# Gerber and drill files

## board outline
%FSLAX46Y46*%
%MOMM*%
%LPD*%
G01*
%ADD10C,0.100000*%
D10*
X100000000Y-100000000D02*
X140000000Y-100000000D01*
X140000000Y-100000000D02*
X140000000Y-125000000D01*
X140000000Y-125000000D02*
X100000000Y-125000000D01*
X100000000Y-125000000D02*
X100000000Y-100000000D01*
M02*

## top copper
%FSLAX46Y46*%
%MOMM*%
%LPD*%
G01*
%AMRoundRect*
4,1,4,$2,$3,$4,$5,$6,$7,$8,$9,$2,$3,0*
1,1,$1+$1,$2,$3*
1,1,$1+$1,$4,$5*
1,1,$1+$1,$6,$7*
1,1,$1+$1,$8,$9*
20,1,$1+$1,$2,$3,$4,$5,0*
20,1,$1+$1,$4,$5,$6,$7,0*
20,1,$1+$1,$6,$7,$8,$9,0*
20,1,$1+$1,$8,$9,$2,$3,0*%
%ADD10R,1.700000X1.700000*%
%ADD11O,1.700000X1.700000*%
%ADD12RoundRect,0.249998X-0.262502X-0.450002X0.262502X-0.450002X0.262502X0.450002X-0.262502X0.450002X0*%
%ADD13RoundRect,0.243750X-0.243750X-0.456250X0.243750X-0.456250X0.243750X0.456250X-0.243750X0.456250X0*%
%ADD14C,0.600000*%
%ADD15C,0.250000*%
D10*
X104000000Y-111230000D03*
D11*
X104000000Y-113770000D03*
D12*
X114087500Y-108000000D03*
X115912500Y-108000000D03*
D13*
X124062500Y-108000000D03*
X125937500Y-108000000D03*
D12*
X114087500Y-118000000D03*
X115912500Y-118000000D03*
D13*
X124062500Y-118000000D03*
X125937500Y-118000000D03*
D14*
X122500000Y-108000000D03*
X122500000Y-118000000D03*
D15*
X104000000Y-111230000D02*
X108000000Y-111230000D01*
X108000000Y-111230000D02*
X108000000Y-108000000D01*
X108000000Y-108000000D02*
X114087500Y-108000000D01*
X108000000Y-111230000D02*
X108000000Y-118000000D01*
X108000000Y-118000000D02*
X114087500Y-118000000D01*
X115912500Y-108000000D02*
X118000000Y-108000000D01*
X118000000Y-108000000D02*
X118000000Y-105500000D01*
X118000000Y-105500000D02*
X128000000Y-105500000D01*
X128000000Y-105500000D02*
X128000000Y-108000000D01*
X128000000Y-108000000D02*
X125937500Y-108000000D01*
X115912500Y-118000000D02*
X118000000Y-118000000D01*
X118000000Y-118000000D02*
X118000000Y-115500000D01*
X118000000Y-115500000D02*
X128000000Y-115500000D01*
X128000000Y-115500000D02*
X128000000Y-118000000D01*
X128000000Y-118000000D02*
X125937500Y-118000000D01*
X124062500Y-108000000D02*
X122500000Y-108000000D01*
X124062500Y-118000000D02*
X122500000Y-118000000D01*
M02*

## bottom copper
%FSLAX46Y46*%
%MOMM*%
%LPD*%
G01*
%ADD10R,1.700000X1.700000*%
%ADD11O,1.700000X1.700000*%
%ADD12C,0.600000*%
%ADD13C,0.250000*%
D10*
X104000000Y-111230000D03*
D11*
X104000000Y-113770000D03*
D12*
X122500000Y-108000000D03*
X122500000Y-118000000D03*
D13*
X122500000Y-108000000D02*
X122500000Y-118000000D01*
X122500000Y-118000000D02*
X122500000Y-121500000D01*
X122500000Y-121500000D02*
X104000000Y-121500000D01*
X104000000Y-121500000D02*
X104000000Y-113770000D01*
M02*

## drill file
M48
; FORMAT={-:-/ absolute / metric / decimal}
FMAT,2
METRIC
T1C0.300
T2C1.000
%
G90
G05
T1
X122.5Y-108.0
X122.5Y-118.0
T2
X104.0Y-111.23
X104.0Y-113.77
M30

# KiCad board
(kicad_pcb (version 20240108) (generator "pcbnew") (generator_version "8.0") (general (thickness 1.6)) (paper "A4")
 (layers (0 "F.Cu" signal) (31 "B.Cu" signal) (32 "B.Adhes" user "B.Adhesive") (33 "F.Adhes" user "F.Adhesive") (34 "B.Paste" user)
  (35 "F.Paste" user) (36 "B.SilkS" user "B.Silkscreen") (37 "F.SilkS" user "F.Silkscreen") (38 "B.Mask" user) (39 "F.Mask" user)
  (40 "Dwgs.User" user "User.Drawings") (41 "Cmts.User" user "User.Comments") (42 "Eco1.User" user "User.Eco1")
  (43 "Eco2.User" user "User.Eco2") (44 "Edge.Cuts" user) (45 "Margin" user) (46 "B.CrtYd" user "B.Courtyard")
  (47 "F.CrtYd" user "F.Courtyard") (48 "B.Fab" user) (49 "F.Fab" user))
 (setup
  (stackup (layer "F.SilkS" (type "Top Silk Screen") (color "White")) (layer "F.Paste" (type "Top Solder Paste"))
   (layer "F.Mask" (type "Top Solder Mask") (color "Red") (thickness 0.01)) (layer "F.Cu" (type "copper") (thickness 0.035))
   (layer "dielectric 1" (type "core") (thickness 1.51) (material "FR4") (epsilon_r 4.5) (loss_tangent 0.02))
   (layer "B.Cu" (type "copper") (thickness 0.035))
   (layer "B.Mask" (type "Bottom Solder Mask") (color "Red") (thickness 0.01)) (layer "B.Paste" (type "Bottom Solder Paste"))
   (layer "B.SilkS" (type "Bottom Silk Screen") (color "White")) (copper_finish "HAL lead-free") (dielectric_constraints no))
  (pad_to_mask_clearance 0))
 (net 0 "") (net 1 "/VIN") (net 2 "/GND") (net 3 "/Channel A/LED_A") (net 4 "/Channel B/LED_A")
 (gr_line (start 100 100) (end 140 100) (stroke (width 0.1) (type default)) (layer "Edge.Cuts"))
 (gr_line (start 140 100) (end 140 125) (stroke (width 0.1) (type default)) (layer "Edge.Cuts"))
 (gr_line (start 140 125) (end 100 125) (stroke (width 0.1) (type default)) (layer "Edge.Cuts"))
 (gr_line (start 100 125) (end 100 100) (stroke (width 0.1) (type default)) (layer "Edge.Cuts"))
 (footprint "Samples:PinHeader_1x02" (layer "F.Cu") (at 104 111.23)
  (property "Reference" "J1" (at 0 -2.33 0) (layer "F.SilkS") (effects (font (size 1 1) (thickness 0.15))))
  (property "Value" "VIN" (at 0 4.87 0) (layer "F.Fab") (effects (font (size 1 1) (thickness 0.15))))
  (pad "1" thru_hole rect (at 0 0) (size 1.7 1.7) (drill 1) (layers "*.Cu" "*.Mask") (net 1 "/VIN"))
  (pad "2" thru_hole oval (at 0 2.54) (size 1.7 1.7) (drill 1) (layers "*.Cu" "*.Mask") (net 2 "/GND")))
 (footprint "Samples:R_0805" (layer "F.Cu") (at 115 108)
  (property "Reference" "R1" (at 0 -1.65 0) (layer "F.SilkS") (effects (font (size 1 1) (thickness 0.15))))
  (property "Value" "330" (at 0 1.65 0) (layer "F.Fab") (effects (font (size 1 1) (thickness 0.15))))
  (pad "1" smd roundrect (at -0.9125 0) (size 1.025 1.4) (layers "F.Cu" "F.Paste" "F.Mask") (roundrect_rratio 0.2439) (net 1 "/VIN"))
  (pad "2" smd roundrect (at 0.9125 0) (size 1.025 1.4) (layers "F.Cu" "F.Paste" "F.Mask") (roundrect_rratio 0.2439)
   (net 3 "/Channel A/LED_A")))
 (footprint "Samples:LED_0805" (layer "F.Cu") (at 125 108)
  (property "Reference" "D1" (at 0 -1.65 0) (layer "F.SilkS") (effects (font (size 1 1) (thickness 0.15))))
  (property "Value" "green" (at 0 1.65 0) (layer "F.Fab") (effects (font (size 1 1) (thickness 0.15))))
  (pad "1" smd roundrect (at -0.9375 0) (size 0.975 1.4) (layers "F.Cu" "F.Paste" "F.Mask") (roundrect_rratio 0.25) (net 2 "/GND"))
  (pad "2" smd roundrect (at 0.9375 0) (size 0.975 1.4) (layers "F.Cu" "F.Paste" "F.Mask") (roundrect_rratio 0.25)
   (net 3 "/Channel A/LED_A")))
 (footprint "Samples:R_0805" (layer "F.Cu") (at 115 118)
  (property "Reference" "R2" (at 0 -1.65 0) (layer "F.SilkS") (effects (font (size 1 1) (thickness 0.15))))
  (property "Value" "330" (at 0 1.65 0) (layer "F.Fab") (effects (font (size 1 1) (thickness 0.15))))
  (pad "1" smd roundrect (at -0.9125 0) (size 1.025 1.4) (layers "F.Cu" "F.Paste" "F.Mask") (roundrect_rratio 0.2439) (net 1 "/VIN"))
  (pad "2" smd roundrect (at 0.9125 0) (size 1.025 1.4) (layers "F.Cu" "F.Paste" "F.Mask") (roundrect_rratio 0.2439)
   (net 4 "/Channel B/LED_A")))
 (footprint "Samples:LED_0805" (layer "F.Cu") (at 125 118)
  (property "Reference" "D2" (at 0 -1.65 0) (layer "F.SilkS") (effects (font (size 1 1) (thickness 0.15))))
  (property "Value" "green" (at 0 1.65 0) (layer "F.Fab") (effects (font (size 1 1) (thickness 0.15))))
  (pad "1" smd roundrect (at -0.9375 0) (size 0.975 1.4) (layers "F.Cu" "F.Paste" "F.Mask") (roundrect_rratio 0.25) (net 2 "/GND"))
  (pad "2" smd roundrect (at 0.9375 0) (size 0.975 1.4) (layers "F.Cu" "F.Paste" "F.Mask") (roundrect_rratio 0.25)
   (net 4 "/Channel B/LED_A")))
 (segment (start 104 111.23) (end 108 111.23) (width 0.25) (layer "F.Cu") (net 1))
 (segment (start 108 111.23) (end 108 108) (width 0.25) (layer "F.Cu") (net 1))
 (segment (start 108 108) (end 114.0875 108) (width 0.25) (layer "F.Cu") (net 1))
 (segment (start 108 111.23) (end 108 118) (width 0.25) (layer "F.Cu") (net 1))
 (segment (start 108 118) (end 114.0875 118) (width 0.25) (layer "F.Cu") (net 1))
 (segment (start 115.9125 108) (end 118 108) (width 0.25) (layer "F.Cu") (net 3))
 (segment (start 118 108) (end 118 105.5) (width 0.25) (layer "F.Cu") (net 3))
 (segment (start 118 105.5) (end 128 105.5) (width 0.25) (layer "F.Cu") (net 3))
 (segment (start 128 105.5) (end 128 108) (width 0.25) (layer "F.Cu") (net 3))
 (segment (start 128 108) (end 125.9375 108) (width 0.25) (layer "F.Cu") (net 3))
 (segment (start 115.9125 118) (end 118 118) (width 0.25) (layer "F.Cu") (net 4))
 (segment (start 118 118) (end 118 115.5) (width 0.25) (layer "F.Cu") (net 4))
 (segment (start 118 115.5) (end 128 115.5) (width 0.25) (layer "F.Cu") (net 4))
 (segment (start 128 115.5) (end 128 118) (width 0.25) (layer "F.Cu") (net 4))
 (segment (start 128 118) (end 125.9375 118) (width 0.25) (layer "F.Cu") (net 4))
 (segment (start 124.0625 108) (end 122.5 108) (width 0.25) (layer "F.Cu") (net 2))
 (segment (start 124.0625 118) (end 122.5 118) (width 0.25) (layer "F.Cu") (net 2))
 (segment (start 122.5 108) (end 122.5 118) (width 0.25) (layer "B.Cu") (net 2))
 (segment (start 122.5 118) (end 122.5 121.5) (width 0.25) (layer "B.Cu") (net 2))
 (segment (start 122.5 121.5) (end 104 121.5) (width 0.25) (layer "B.Cu") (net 2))
 (segment (start 104 121.5) (end 104 113.77) (width 0.25) (layer "B.Cu") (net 2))
 (via (at 122.5 108) (size 0.6) (drill 0.3) (layers "F.Cu" "B.Cu") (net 2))
 (via (at 122.5 118) (size 0.6) (drill 0.3) (layers "F.Cu" "B.Cu") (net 2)))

